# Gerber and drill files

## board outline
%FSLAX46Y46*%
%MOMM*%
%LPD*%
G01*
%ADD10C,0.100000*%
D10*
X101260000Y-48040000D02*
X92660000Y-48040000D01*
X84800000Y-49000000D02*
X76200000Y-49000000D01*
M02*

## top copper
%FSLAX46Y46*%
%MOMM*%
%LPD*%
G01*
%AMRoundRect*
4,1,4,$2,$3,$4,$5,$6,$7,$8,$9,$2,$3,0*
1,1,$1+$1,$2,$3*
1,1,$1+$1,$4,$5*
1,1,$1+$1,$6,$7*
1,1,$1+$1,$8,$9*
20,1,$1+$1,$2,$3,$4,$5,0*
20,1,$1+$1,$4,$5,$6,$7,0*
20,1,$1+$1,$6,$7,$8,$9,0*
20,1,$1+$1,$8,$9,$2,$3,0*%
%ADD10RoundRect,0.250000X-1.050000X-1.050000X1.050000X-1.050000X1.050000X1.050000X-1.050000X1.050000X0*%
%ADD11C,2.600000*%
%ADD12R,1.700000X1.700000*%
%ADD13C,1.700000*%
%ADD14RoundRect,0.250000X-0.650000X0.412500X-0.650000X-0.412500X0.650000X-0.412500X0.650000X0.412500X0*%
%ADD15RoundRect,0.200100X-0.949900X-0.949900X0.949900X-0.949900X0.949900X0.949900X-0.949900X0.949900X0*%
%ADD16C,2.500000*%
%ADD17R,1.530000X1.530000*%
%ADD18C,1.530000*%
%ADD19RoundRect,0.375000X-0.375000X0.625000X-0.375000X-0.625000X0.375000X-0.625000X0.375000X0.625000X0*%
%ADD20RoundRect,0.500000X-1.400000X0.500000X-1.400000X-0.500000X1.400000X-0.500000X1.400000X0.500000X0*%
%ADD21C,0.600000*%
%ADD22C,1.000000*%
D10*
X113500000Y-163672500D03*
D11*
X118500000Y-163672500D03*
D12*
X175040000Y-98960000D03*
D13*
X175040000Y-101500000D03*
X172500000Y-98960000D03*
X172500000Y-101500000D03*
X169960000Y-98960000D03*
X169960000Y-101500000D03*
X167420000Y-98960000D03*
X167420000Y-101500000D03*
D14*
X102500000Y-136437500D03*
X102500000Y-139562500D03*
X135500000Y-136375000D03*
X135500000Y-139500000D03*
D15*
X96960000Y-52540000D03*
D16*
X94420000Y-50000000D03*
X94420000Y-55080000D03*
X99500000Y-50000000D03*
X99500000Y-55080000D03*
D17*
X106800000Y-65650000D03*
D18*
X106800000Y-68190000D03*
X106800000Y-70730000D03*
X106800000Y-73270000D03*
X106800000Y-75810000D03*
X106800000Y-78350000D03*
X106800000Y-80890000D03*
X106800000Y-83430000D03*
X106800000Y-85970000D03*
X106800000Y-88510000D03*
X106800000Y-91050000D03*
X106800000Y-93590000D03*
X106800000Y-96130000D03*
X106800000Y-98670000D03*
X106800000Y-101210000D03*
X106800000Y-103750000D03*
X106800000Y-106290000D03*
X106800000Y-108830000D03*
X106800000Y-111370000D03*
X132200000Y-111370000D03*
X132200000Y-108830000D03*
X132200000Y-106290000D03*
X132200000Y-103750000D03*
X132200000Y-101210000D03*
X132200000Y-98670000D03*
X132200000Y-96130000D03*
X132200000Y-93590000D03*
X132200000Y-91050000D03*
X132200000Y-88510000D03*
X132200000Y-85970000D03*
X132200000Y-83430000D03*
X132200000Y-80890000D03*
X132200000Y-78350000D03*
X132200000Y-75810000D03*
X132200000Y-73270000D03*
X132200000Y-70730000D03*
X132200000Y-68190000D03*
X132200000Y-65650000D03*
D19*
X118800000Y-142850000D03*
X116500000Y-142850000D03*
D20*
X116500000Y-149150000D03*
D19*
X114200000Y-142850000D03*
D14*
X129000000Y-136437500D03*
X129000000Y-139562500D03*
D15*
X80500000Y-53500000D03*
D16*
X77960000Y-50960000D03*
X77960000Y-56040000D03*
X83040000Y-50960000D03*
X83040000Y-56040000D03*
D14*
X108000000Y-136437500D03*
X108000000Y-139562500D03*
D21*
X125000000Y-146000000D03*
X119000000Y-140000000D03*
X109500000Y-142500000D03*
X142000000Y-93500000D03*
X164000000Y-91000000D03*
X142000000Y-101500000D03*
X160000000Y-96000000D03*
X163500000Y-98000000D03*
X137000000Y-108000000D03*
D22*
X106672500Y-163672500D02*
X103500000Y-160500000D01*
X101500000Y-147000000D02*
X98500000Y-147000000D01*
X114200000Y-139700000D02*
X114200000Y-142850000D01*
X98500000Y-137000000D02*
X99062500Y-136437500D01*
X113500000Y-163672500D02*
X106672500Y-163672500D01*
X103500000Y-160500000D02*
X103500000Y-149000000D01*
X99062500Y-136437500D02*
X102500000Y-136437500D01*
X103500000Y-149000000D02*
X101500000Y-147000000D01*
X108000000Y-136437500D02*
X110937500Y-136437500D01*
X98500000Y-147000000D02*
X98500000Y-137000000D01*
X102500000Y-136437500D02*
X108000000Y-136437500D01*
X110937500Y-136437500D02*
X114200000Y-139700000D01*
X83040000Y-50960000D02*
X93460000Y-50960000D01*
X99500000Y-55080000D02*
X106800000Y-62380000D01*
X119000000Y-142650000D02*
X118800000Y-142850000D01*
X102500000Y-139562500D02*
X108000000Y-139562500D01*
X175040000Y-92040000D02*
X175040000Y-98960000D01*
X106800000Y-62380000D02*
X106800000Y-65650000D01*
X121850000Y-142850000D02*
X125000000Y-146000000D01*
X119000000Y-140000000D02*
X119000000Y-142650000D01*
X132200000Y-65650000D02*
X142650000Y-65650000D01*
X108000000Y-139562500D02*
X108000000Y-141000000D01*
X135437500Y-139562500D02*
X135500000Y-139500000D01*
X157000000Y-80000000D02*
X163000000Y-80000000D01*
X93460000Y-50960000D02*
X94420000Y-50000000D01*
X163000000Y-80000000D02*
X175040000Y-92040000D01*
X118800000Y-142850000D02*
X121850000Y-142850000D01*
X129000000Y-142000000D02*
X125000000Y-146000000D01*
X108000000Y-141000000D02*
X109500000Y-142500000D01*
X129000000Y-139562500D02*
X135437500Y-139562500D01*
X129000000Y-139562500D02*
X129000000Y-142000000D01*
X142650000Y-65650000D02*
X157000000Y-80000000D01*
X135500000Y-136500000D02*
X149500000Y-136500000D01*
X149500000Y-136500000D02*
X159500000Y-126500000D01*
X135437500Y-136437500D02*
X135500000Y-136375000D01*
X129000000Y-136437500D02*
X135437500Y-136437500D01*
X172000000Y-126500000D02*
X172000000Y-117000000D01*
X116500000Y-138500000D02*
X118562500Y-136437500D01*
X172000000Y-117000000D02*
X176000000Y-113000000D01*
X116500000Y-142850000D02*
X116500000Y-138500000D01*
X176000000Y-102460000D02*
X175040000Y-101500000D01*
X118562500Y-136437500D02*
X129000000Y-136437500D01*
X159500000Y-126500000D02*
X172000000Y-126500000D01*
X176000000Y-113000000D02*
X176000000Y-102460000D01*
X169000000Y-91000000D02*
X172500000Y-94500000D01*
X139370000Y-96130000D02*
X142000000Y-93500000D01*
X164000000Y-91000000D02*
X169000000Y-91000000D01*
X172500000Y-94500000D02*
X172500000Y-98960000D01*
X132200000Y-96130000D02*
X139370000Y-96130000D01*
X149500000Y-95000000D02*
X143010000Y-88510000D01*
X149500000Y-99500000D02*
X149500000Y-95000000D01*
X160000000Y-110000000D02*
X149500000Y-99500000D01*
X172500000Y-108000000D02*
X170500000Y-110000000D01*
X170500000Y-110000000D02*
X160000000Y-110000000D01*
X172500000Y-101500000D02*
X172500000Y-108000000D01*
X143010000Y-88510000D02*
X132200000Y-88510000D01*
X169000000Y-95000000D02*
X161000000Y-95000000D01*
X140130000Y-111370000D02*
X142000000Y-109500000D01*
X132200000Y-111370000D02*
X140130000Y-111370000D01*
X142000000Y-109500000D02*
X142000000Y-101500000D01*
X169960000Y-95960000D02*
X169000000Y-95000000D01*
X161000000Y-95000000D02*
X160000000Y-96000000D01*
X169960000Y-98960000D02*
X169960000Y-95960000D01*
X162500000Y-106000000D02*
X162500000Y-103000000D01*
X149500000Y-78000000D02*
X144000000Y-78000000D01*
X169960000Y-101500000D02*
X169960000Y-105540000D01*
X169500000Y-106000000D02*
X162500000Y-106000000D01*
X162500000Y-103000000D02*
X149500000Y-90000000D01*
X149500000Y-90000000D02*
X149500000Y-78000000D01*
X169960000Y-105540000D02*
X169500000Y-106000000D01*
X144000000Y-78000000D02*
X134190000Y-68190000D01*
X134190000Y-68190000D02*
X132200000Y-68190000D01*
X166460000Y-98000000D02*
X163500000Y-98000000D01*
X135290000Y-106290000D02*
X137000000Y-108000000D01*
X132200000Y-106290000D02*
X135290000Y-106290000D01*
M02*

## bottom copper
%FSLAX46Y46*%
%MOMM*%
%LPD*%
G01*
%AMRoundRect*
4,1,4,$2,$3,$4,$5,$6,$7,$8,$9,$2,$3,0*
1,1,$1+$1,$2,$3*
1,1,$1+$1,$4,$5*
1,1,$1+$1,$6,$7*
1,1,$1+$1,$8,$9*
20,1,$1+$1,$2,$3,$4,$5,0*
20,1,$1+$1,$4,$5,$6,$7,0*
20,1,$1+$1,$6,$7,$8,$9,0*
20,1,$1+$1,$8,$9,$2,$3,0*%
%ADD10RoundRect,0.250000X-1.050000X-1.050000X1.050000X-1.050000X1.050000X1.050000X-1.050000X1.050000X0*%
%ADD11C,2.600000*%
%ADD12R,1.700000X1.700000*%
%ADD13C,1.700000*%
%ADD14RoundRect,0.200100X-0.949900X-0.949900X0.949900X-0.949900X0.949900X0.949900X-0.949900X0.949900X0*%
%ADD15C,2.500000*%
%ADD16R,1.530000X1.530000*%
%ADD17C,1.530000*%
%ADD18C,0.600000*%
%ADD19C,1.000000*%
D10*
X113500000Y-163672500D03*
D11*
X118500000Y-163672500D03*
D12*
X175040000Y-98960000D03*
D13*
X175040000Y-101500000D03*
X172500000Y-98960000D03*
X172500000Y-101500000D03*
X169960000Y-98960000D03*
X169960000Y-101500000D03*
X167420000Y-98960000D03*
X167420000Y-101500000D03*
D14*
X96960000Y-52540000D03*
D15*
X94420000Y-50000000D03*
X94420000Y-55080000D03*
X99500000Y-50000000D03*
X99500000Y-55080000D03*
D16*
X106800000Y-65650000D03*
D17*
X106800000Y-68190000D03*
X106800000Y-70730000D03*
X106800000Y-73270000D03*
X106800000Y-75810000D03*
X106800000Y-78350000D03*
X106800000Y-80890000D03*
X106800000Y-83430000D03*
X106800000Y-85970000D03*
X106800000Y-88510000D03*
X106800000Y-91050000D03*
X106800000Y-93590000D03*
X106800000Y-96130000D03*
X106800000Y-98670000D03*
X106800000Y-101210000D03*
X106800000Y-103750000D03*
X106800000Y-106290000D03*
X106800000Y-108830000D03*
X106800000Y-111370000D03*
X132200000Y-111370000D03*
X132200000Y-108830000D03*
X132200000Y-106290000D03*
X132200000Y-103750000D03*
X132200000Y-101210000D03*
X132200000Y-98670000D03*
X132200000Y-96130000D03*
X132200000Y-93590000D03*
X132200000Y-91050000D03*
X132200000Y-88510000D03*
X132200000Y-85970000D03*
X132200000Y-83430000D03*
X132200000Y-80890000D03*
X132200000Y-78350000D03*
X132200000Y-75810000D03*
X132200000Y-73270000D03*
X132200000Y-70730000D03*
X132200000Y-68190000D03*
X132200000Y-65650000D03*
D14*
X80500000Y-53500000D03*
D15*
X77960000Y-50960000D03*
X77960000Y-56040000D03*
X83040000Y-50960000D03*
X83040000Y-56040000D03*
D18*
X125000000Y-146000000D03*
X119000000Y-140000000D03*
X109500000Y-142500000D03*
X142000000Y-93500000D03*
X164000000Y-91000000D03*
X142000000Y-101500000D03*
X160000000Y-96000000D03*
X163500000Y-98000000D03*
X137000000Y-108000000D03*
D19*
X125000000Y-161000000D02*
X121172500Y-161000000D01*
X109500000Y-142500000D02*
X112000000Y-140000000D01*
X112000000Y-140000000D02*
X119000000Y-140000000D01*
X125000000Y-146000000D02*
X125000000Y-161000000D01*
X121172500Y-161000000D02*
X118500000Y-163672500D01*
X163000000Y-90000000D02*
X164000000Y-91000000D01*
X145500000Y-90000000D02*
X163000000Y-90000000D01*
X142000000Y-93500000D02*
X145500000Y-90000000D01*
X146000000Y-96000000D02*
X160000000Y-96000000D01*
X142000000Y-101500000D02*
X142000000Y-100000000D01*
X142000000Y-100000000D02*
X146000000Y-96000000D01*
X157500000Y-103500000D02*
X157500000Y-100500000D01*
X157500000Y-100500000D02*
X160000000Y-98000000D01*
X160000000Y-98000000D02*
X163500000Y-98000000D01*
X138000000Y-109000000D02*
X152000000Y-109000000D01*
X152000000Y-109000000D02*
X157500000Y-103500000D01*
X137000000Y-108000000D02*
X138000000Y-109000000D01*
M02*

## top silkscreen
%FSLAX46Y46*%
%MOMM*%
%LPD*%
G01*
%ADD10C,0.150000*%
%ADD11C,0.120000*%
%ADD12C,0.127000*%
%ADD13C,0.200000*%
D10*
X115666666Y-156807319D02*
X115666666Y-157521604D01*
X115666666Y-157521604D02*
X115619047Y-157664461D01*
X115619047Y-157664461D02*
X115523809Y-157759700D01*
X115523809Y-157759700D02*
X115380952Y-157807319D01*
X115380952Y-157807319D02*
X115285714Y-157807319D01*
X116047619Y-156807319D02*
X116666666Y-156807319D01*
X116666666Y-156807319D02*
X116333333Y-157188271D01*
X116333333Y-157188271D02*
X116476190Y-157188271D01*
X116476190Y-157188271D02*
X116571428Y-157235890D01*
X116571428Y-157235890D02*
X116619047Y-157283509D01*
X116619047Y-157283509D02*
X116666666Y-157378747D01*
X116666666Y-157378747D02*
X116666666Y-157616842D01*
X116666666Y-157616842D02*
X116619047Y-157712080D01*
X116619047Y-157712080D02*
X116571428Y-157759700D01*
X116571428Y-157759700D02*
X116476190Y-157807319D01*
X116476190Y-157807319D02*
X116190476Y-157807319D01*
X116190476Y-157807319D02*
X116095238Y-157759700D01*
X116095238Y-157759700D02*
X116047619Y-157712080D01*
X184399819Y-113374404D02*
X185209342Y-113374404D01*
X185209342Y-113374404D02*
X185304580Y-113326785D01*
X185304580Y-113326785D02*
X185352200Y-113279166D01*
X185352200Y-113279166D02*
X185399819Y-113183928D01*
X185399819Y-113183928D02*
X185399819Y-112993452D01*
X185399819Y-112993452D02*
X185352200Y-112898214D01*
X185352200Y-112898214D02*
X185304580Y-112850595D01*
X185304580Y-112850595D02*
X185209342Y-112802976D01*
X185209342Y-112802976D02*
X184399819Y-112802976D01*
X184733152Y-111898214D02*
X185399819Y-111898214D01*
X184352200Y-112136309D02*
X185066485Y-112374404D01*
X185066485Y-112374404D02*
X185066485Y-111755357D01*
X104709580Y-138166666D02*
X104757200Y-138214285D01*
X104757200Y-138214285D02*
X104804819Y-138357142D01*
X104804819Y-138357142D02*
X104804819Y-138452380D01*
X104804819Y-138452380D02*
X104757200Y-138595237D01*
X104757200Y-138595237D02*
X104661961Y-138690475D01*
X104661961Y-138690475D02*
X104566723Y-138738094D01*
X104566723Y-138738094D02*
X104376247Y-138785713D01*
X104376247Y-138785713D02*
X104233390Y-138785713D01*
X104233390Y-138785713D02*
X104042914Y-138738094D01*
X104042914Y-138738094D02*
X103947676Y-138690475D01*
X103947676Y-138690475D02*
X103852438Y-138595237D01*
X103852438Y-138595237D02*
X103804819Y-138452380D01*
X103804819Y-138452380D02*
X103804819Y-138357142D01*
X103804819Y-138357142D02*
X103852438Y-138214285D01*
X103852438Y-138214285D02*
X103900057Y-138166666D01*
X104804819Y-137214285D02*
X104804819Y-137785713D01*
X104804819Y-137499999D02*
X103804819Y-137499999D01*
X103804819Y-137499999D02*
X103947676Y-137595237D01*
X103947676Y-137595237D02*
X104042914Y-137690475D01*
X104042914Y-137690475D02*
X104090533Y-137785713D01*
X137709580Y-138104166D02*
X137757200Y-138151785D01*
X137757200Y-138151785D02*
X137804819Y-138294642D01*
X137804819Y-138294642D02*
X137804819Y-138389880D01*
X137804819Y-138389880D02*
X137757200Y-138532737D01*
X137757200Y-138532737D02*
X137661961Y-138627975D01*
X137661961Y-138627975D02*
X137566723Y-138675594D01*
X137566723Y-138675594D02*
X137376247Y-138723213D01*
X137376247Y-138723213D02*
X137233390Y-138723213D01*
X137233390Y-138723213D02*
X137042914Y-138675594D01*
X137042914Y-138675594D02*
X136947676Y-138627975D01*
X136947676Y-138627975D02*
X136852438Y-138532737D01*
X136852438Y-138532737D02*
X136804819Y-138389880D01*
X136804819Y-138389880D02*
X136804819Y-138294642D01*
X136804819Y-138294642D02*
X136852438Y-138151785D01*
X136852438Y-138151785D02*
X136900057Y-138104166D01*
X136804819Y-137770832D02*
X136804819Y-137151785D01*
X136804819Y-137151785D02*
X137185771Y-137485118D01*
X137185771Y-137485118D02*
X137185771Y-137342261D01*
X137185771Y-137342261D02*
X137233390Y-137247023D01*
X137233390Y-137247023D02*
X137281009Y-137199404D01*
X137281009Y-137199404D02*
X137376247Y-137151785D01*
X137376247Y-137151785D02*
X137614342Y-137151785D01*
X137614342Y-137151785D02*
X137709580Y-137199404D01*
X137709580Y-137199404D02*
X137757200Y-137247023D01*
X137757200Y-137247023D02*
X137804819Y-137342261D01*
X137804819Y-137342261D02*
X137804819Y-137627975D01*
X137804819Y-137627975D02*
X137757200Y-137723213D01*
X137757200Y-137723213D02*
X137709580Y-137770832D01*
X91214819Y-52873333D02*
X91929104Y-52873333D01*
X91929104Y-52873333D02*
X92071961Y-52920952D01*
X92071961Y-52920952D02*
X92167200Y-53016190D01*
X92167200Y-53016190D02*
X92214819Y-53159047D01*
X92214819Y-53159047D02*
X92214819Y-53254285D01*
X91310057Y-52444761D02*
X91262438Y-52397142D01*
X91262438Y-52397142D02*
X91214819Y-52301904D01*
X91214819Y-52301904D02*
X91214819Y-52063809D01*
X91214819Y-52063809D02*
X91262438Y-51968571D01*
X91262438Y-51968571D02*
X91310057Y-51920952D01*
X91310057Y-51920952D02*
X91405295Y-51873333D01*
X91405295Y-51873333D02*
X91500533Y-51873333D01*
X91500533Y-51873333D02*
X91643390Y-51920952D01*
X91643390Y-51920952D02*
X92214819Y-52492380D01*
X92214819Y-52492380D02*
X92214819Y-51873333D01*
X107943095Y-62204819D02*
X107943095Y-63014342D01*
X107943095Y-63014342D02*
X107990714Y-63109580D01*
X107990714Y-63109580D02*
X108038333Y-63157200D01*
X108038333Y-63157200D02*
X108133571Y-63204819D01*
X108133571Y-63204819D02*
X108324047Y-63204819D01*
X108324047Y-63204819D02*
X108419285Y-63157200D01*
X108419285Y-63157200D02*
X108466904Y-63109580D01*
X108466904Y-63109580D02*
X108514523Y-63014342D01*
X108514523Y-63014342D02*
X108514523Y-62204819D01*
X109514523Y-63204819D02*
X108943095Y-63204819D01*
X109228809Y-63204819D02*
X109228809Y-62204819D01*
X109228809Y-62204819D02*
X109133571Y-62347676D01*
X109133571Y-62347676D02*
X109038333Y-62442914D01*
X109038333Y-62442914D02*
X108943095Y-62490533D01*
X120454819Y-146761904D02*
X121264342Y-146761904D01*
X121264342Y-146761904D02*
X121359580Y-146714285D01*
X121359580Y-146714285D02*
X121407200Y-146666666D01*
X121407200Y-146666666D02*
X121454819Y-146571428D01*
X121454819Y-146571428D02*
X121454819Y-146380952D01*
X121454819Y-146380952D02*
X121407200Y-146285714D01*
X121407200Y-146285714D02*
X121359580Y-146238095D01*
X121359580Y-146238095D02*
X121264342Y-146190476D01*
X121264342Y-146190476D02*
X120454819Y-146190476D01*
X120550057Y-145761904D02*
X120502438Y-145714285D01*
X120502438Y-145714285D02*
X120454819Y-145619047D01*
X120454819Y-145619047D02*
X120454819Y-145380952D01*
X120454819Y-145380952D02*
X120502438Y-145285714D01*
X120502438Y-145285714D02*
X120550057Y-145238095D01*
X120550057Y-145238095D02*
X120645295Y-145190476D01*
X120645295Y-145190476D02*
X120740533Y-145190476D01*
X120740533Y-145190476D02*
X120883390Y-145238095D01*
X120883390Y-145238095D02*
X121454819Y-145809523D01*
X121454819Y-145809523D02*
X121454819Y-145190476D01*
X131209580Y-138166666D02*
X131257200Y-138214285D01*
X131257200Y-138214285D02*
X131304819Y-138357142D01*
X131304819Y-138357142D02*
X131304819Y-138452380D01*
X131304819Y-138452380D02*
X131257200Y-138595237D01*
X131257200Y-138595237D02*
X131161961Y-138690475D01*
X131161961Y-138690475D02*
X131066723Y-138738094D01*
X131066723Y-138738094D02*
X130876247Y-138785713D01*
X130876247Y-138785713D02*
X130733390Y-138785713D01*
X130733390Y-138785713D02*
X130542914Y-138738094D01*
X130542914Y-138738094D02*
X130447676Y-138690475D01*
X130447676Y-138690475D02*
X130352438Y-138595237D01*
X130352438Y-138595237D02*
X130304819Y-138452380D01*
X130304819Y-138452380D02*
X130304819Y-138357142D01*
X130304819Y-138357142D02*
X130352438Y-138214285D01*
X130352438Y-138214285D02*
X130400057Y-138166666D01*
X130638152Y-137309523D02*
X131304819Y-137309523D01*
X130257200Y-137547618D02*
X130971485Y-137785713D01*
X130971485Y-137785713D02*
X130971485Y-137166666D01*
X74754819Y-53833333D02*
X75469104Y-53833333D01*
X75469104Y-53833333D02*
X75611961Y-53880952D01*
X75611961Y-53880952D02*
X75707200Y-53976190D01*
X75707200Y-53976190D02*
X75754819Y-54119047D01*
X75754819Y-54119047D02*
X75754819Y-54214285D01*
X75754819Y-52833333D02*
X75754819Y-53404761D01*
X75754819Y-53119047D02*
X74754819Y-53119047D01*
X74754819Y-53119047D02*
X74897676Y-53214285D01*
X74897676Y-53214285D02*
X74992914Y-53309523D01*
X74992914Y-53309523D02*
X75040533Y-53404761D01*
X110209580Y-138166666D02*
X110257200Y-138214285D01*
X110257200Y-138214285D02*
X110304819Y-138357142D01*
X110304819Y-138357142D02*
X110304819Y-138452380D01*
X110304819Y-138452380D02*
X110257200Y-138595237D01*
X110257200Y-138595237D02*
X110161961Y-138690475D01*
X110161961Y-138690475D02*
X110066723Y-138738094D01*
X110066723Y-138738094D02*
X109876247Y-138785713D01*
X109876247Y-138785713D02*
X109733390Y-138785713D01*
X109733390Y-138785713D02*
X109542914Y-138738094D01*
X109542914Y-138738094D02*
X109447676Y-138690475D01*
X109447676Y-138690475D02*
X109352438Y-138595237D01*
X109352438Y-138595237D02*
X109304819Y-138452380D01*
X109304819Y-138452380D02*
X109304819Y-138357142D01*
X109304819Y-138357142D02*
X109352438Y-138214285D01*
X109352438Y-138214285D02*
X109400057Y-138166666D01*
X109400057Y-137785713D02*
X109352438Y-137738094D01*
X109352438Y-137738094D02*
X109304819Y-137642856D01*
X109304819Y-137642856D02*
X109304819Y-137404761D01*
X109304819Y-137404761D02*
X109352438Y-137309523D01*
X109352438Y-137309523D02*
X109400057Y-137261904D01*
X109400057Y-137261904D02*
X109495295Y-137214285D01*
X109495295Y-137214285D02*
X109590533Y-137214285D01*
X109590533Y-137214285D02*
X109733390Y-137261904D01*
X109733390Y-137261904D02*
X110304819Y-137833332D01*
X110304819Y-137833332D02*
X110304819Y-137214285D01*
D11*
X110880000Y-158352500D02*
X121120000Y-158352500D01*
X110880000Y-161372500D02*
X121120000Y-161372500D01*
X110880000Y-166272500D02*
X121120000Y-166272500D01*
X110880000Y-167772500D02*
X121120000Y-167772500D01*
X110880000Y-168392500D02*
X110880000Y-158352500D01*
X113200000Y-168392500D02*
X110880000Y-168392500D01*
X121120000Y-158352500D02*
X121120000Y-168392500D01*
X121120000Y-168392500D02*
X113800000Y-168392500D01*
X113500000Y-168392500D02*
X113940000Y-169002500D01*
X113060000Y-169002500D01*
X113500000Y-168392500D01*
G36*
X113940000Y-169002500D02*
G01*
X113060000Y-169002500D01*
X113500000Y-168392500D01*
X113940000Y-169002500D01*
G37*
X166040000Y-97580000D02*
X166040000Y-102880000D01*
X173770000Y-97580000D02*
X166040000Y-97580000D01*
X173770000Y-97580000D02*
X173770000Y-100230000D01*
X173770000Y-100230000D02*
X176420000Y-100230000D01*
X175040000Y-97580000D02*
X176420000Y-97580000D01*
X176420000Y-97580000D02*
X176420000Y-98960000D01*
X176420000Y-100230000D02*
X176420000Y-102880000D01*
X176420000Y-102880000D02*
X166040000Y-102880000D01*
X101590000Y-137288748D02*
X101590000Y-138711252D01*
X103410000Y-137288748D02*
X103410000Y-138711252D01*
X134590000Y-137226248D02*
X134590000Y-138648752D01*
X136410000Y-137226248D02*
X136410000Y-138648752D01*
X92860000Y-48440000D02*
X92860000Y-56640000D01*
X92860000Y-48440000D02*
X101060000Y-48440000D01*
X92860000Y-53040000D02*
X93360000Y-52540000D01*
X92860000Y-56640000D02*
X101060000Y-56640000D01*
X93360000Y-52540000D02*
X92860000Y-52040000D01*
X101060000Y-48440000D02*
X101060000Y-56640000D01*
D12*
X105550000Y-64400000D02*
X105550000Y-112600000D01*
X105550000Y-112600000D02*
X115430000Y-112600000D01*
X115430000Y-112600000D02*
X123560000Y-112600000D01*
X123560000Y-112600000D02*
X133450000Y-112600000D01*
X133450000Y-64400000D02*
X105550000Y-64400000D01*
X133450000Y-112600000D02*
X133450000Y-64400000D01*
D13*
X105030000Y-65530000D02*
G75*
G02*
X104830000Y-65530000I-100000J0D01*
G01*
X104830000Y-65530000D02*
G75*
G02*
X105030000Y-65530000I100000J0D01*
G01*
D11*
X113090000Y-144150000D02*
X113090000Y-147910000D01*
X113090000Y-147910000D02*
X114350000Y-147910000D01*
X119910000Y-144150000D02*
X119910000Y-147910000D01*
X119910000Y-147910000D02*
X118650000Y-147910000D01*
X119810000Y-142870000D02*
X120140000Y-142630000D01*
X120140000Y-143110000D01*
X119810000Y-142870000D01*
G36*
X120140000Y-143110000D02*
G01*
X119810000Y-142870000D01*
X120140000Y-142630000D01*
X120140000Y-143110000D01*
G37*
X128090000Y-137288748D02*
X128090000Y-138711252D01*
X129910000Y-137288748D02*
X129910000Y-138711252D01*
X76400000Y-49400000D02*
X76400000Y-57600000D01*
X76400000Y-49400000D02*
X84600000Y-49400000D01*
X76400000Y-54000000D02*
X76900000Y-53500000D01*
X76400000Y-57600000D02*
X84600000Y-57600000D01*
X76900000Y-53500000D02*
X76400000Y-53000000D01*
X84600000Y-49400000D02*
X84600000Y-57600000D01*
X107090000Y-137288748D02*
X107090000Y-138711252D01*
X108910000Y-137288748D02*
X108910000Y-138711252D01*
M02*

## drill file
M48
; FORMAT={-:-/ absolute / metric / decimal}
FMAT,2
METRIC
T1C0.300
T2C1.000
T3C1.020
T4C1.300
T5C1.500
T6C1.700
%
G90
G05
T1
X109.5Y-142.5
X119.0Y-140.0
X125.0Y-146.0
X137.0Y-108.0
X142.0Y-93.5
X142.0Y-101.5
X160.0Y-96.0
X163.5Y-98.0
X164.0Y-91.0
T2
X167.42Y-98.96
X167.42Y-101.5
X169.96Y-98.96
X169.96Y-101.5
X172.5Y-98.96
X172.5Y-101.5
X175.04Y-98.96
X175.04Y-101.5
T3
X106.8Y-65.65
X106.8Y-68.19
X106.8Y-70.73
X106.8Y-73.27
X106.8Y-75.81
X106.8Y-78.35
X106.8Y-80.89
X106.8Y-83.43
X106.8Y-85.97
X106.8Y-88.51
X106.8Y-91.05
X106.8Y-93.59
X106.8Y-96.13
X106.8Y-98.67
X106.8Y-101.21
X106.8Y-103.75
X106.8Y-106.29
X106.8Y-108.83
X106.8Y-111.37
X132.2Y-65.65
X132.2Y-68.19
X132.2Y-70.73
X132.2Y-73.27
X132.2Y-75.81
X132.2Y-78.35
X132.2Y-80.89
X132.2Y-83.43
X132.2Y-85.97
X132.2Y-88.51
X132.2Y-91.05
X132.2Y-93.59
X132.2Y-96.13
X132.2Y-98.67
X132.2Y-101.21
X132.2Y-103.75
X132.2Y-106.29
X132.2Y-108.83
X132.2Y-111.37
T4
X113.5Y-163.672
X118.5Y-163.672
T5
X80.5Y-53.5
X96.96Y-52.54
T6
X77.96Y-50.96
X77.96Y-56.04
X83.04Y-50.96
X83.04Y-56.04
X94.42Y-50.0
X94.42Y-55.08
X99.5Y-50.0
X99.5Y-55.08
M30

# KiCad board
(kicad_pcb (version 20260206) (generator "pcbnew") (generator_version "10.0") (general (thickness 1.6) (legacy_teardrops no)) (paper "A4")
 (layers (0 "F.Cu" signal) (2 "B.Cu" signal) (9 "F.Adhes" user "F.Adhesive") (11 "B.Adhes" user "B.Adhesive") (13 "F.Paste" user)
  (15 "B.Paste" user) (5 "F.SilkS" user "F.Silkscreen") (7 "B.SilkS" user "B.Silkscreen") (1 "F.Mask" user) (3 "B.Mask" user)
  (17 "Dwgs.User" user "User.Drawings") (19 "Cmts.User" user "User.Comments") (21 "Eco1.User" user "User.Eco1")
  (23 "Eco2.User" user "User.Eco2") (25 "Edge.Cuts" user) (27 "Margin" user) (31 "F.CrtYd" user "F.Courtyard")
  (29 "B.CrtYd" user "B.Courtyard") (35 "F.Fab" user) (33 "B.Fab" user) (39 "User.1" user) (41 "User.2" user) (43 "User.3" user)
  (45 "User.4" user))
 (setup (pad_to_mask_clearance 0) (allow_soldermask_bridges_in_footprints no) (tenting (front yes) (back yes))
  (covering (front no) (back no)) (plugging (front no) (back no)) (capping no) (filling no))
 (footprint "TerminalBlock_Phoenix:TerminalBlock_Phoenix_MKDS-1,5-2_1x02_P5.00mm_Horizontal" (layer "F.Cu") (at 113.5 163.6725)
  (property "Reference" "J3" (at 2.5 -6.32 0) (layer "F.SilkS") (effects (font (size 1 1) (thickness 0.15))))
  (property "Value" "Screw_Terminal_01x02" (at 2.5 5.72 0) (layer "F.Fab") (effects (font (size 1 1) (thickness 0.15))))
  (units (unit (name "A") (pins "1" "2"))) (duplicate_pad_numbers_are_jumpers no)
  (fp_line (start -2.62 -5.32) (end 7.62 -5.32) (stroke (width 0.12) (type solid)) (layer "F.SilkS"))
  (fp_line (start -2.62 -2.3) (end 7.62 -2.3) (stroke (width 0.12) (type solid)) (layer "F.SilkS"))
  (fp_line (start -2.62 2.6) (end 7.62 2.6) (stroke (width 0.12) (type solid)) (layer "F.SilkS"))
  (fp_line (start -2.62 4.1) (end 7.62 4.1) (stroke (width 0.12) (type solid)) (layer "F.SilkS"))
  (fp_line (start -2.62 4.72) (end -2.62 -5.32) (stroke (width 0.12) (type solid)) (layer "F.SilkS"))
  (fp_line (start -0.3 4.72) (end -2.62 4.72) (stroke (width 0.12) (type solid)) (layer "F.SilkS"))
  (fp_line (start 7.62 -5.32) (end 7.62 4.72) (stroke (width 0.12) (type solid)) (layer "F.SilkS"))
  (fp_line (start 7.62 4.72) (end 0.3 4.72) (stroke (width 0.12) (type solid)) (layer "F.SilkS"))
  (fp_poly (pts (xy 0 4.72) (xy 0.44 5.33) (xy -0.44 5.33)) (stroke (width 0.12) (type solid)) (fill yes) (layer "F.SilkS"))
  (pad "1" thru_hole roundrect (at 0 0) (size 2.6 2.6) (drill 1.3) (layers "*.Cu" "*.Mask") (remove_unused_layers no)
   (roundrect_rratio 0.096154) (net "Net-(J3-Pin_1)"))
  (pad "2" thru_hole circle (at 5 0) (size 2.6 2.6) (drill 1.3) (layers "*.Cu" "*.Mask") (remove_unused_layers no) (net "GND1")))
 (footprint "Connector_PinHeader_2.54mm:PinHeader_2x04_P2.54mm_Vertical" (layer "F.Cu") (at 175.04 98.96 -90)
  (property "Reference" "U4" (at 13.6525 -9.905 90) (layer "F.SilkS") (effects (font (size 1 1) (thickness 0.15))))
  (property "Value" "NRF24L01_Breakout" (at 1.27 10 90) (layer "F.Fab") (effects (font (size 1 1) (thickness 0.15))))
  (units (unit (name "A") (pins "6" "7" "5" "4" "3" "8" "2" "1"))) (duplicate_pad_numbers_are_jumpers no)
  (fp_line (start -1.38 9) (end 3.92 9) (stroke (width 0.12) (type solid)) (layer "F.SilkS"))
  (fp_line (start -1.38 1.27) (end -1.38 9) (stroke (width 0.12) (type solid)) (layer "F.SilkS"))
  (fp_line (start -1.38 1.27) (end 1.27 1.27) (stroke (width 0.12) (type solid)) (layer "F.SilkS"))
  (fp_line (start 1.27 1.27) (end 1.27 -1.38) (stroke (width 0.12) (type solid)) (layer "F.SilkS"))
  (fp_line (start -1.38 0) (end -1.38 -1.38) (stroke (width 0.12) (type solid)) (layer "F.SilkS"))
  (fp_line (start -1.38 -1.38) (end 0 -1.38) (stroke (width 0.12) (type solid)) (layer "F.SilkS"))
  (fp_line (start 1.27 -1.38) (end 3.92 -1.38) (stroke (width 0.12) (type solid)) (layer "F.SilkS"))
  (fp_line (start 3.92 -1.38) (end 3.92 9) (stroke (width 0.12) (type solid)) (layer "F.SilkS"))
  (pad "1" thru_hole rect (at 0 0 270) (size 1.7 1.7) (drill 1) (layers "*.Cu" "*.Mask") (remove_unused_layers no) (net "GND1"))
  (pad "2" thru_hole circle (at 2.54 0 270) (size 1.7 1.7) (drill 1) (layers "*.Cu" "*.Mask") (remove_unused_layers no) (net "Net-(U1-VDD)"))
  (pad "3" thru_hole circle (at 0 2.54 270) (size 1.7 1.7) (drill 1) (layers "*.Cu" "*.Mask") (remove_unused_layers no) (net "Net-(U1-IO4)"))
  (pad "4" thru_hole circle (at 2.54 2.54 270) (size 1.7 1.7) (drill 1) (layers "*.Cu" "*.Mask") (remove_unused_layers no)
   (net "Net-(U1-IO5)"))
  (pad "5" thru_hole circle (at 0 5.08 270) (size 1.7 1.7) (drill 1) (layers "*.Cu" "*.Mask") (remove_unused_layers no)
   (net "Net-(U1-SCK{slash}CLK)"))
  (pad "6" thru_hole circle (at 2.54 5.08 270) (size 1.7 1.7) (drill 1) (layers "*.Cu" "*.Mask") (remove_unused_layers no)
   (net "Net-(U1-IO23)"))
  (pad "7" thru_hole circle (at 0 7.62 270) (size 1.7 1.7) (drill 1) (layers "*.Cu" "*.Mask") (remove_unused_layers no)
   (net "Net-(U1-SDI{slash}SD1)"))
  (pad "8" thru_hole circle (at 2.54 7.62 270) (size 1.7 1.7) (drill 1) (layers "*.Cu" "*.Mask") (remove_unused_layers no)
   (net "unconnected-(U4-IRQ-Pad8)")))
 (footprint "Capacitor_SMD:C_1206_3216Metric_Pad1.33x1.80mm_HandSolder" (layer "F.Cu") (at 102.5 138 -90)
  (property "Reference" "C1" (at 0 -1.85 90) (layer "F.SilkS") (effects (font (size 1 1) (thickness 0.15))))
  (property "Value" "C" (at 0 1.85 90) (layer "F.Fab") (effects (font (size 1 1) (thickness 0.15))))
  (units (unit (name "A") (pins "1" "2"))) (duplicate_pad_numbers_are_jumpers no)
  (fp_line (start -0.711252 0.91) (end 0.711252 0.91) (stroke (width 0.12) (type solid)) (layer "F.SilkS"))
  (fp_line (start -0.711252 -0.91) (end 0.711252 -0.91) (stroke (width 0.12) (type solid)) (layer "F.SilkS"))
  (pad "1" smd roundrect (at -1.5625 0 270) (size 1.325 1.8) (layers "F.Cu" "F.Mask" "F.Paste") (roundrect_rratio 0.188679)
   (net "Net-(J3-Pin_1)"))
  (pad "2" smd roundrect (at 1.5625 0 270) (size 1.325 1.8) (layers "F.Cu" "F.Mask" "F.Paste") (roundrect_rratio 0.188679) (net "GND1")))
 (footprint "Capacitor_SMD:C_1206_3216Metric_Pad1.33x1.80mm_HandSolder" (layer "F.Cu") (at 135.5 137.9375 -90)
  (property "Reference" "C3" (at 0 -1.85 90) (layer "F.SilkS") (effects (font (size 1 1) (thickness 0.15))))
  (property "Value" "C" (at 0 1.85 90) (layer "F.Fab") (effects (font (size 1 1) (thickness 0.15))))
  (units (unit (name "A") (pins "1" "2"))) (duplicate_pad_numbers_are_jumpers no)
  (fp_line (start -0.711252 0.91) (end 0.711252 0.91) (stroke (width 0.12) (type solid)) (layer "F.SilkS"))
  (fp_line (start -0.711252 -0.91) (end 0.711252 -0.91) (stroke (width 0.12) (type solid)) (layer "F.SilkS"))
  (pad "1" smd roundrect (at -1.5625 0 270) (size 1.325 1.8) (layers "F.Cu" "F.Mask" "F.Paste") (roundrect_rratio 0.188679)
   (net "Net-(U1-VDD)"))
  (pad "2" smd roundrect (at 1.5625 0 270) (size 1.325 1.8) (layers "F.Cu" "F.Mask" "F.Paste") (roundrect_rratio 0.188679) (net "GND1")))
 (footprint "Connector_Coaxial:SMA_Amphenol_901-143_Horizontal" (layer "F.Cu") (at 96.96 52.54)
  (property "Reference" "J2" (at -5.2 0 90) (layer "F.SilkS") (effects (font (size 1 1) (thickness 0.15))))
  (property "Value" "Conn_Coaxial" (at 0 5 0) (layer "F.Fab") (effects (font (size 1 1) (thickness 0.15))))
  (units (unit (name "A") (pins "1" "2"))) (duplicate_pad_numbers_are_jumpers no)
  (fp_line (start -4.1 -4.1) (end -4.1 4.1) (stroke (width 0.12) (type solid)) (layer "F.SilkS"))
  (fp_line (start -4.1 -4.1) (end 4.1 -4.1) (stroke (width 0.12) (type solid)) (layer "F.SilkS"))
  (fp_line (start -4.1 0.5) (end -3.6 0) (stroke (width 0.12) (type solid)) (layer "F.SilkS"))
  (fp_line (start -4.1 4.1) (end 4.1 4.1) (stroke (width 0.12) (type solid)) (layer "F.SilkS"))
  (fp_line (start -3.6 0) (end -4.1 -0.5) (stroke (width 0.12) (type solid)) (layer "F.SilkS"))
  (fp_line (start 4.1 -4.1) (end 4.1 4.1) (stroke (width 0.12) (type solid)) (layer "F.SilkS"))
  (fp_line (start 4.3 -4.5) (end -4.3 -4.5) (stroke (width 0.1) (type solid)) (layer "Edge.Cuts"))
  (pad "1" thru_hole roundrect (at 0 0) (size 2.3 2.3) (drill 1.5) (layers "*.Cu" "*.Mask") (remove_unused_layers yes) (keep_end_layers yes)
   (zone_layer_connections) (roundrect_rratio 0.087) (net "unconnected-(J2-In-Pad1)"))
  (pad "2" thru_hole circle (at -2.54 -2.54) (size 2.5 2.5) (drill 1.7) (layers "*.Cu" "*.Mask") (remove_unused_layers yes)
   (keep_end_layers yes) (zone_layer_connections) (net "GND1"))
  (pad "2" thru_hole circle (at -2.54 2.54) (size 2.5 2.5) (drill 1.7) (layers "*.Cu" "*.Mask") (remove_unused_layers yes)
   (keep_end_layers yes) (zone_layer_connections) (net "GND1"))
  (pad "2" thru_hole circle (at 2.54 -2.54) (size 2.5 2.5) (drill 1.7) (layers "*.Cu" "*.Mask") (remove_unused_layers yes)
   (keep_end_layers yes) (zone_layer_connections) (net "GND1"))
  (pad "2" thru_hole circle (at 2.54 2.54) (size 2.5 2.5) (drill 1.7) (layers "*.Cu" "*.Mask") (remove_unused_layers yes)
   (keep_end_layers yes) (zone_layer_connections) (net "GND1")))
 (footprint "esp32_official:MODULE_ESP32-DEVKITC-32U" (layer "F.Cu") (at 119.5 88.5)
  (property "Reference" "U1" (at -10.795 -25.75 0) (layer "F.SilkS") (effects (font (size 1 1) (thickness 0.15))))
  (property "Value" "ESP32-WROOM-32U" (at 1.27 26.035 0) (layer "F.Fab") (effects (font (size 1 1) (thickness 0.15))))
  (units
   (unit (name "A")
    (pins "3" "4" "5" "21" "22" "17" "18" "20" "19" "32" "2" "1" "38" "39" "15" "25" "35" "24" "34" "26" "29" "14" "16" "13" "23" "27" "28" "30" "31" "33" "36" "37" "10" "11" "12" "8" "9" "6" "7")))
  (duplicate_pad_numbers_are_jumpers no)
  (fp_line (start -13.95 -24.1) (end -13.95 24.1) (stroke (width 0.127) (type solid)) (layer "F.SilkS"))
  (fp_line (start -13.95 24.1) (end -4.07 24.1) (stroke (width 0.127) (type solid)) (layer "F.SilkS"))
  (fp_line (start -4.07 24.1) (end 4.06 24.1) (stroke (width 0.127) (type solid)) (layer "F.SilkS"))
  (fp_line (start 4.06 24.1) (end 13.95 24.1) (stroke (width 0.127) (type solid)) (layer "F.SilkS"))
  (fp_line (start 13.95 -24.1) (end -13.95 -24.1) (stroke (width 0.127) (type solid)) (layer "F.SilkS"))
  (fp_line (start 13.95 24.1) (end 13.95 -24.1) (stroke (width 0.127) (type solid)) (layer "F.SilkS"))
  (fp_circle (center -14.57 -22.97) (end -14.47 -22.97) (stroke (width 0.2) (type solid)) (fill no) (layer "F.SilkS"))
  (pad "1" thru_hole rect (at -12.7 -22.85) (size 1.53 1.53) (drill 1.02) (layers "*.Cu" "*.Mask") (remove_unused_layers no) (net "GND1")
   (solder_mask_margin 0.102))
  (pad "2" thru_hole circle (at -12.7 -20.31) (size 1.53 1.53) (drill 1.02) (layers "*.Cu" "*.Mask") (remove_unused_layers no)
   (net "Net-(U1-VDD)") (solder_mask_margin 0.102))
  (pad "3" thru_hole circle (at -12.7 -17.77) (size 1.53 1.53) (drill 1.02) (layers "*.Cu" "*.Mask") (remove_unused_layers no)
   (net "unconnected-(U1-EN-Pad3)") (solder_mask_margin 0.102))
  (pad "4" thru_hole circle (at -12.7 -15.23) (size 1.53 1.53) (drill 1.02) (layers "*.Cu" "*.Mask") (remove_unused_layers no)
   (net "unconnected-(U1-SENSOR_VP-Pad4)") (solder_mask_margin 0.102))
  (pad "5" thru_hole circle (at -12.7 -12.69) (size 1.53 1.53) (drill 1.02) (layers "*.Cu" "*.Mask") (remove_unused_layers no)
   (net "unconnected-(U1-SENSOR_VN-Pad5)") (solder_mask_margin 0.102))
  (pad "6" thru_hole circle (at -12.7 -10.15) (size 1.53 1.53) (drill 1.02) (layers "*.Cu" "*.Mask") (remove_unused_layers no)
   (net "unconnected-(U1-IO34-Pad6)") (solder_mask_margin 0.102))
  (pad "7" thru_hole circle (at -12.7 -7.61) (size 1.53 1.53) (drill 1.02) (layers "*.Cu" "*.Mask") (remove_unused_layers no)
   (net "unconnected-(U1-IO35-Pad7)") (solder_mask_margin 0.102))
  (pad "8" thru_hole circle (at -12.7 -5.07) (size 1.53 1.53) (drill 1.02) (layers "*.Cu" "*.Mask") (remove_unused_layers no)
   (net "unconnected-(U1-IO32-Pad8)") (solder_mask_margin 0.102))
  (pad "9" thru_hole circle (at -12.7 -2.53) (size 1.53 1.53) (drill 1.02) (layers "*.Cu" "*.Mask") (remove_unused_layers no)
   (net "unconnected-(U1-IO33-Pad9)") (solder_mask_margin 0.102))
  (pad "10" thru_hole circle (at -12.7 0.01) (size 1.53 1.53) (drill 1.02) (layers "*.Cu" "*.Mask") (remove_unused_layers no)
   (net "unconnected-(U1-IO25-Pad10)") (solder_mask_margin 0.102))
  (pad "11" thru_hole circle (at -12.7 2.55) (size 1.53 1.53) (drill 1.02) (layers "*.Cu" "*.Mask") (remove_unused_layers no)
   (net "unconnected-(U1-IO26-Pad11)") (solder_mask_margin 0.102))
  (pad "12" thru_hole circle (at -12.7 5.09) (size 1.53 1.53) (drill 1.02) (layers "*.Cu" "*.Mask") (remove_unused_layers no)
   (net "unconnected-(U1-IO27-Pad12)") (solder_mask_margin 0.102))
  (pad "13" thru_hole circle (at -12.7 7.63) (size 1.53 1.53) (drill 1.02) (layers "*.Cu" "*.Mask") (remove_unused_layers no)
   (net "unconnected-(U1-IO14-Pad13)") (solder_mask_margin 0.102))
  (pad "14" thru_hole circle (at -12.7 10.17) (size 1.53 1.53) (drill 1.02) (layers "*.Cu" "*.Mask") (remove_unused_layers no)
   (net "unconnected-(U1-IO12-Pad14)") (solder_mask_margin 0.102))
  (pad "15" thru_hole circle (at -12.7 12.71) (size 1.53 1.53) (drill 1.02) (layers "*.Cu" "*.Mask") (remove_unused_layers no) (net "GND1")
   (solder_mask_margin 0.102))
  (pad "16" thru_hole circle (at -12.7 15.25) (size 1.53 1.53) (drill 1.02) (layers "*.Cu" "*.Mask") (remove_unused_layers no)
   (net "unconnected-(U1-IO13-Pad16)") (solder_mask_margin 0.102))
  (pad "17" thru_hole circle (at -12.7 17.79) (size 1.53 1.53) (drill 1.02) (layers "*.Cu" "*.Mask") (remove_unused_layers no)
   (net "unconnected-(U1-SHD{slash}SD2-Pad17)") (solder_mask_margin 0.102))
  (pad "18" thru_hole circle (at -12.7 20.33) (size 1.53 1.53) (drill 1.02) (layers "*.Cu" "*.Mask") (remove_unused_layers no)
   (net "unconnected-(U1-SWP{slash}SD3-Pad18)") (solder_mask_margin 0.102))
  (pad "19" thru_hole circle (at -12.7 22.87) (size 1.53 1.53) (drill 1.02) (layers "*.Cu" "*.Mask") (remove_unused_layers no)
   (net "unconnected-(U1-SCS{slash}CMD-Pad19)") (solder_mask_margin 0.102))
  (pad "20" thru_hole circle (at 12.7 22.87) (size 1.53 1.53) (drill 1.02) (layers "*.Cu" "*.Mask") (remove_unused_layers no)
   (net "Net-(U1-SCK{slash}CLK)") (solder_mask_margin 0.102))
  (pad "21" thru_hole circle (at 12.7 20.33) (size 1.53 1.53) (drill 1.02) (layers "*.Cu" "*.Mask") (remove_unused_layers no)
   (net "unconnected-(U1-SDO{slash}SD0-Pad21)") (solder_mask_margin 0.102))
  (pad "22" thru_hole circle (at 12.7 17.79) (size 1.53 1.53) (drill 1.02) (layers "*.Cu" "*.Mask") (remove_unused_layers no)
   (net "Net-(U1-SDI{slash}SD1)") (solder_mask_margin 0.102))
  (pad "23" thru_hole circle (at 12.7 15.25) (size 1.53 1.53) (drill 1.02) (layers "*.Cu" "*.Mask") (remove_unused_layers no)
   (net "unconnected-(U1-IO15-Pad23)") (solder_mask_margin 0.102))
  (pad "24" thru_hole circle (at 12.7 12.71) (size 1.53 1.53) (drill 1.02) (layers "*.Cu" "*.Mask") (remove_unused_layers no)
   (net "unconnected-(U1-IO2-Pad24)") (solder_mask_margin 0.102))
  (pad "25" thru_hole circle (at 12.7 10.17) (size 1.53 1.53) (drill 1.02) (layers "*.Cu" "*.Mask") (remove_unused_layers no)
   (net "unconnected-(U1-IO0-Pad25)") (solder_mask_margin 0.102))
  (pad "26" thru_hole circle (at 12.7 7.63) (size 1.53 1.53) (drill 1.02) (layers "*.Cu" "*.Mask") (remove_unused_layers no)
   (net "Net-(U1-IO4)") (solder_mask_margin 0.102))
  (pad "27" thru_hole circle (at 12.7 5.09) (size 1.53 1.53) (drill 1.02) (layers "*.Cu" "*.Mask") (remove_unused_layers no)
   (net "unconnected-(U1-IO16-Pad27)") (solder_mask_margin 0.102))
  (pad "28" thru_hole circle (at 12.7 2.55) (size 1.53 1.53) (drill 1.02) (layers "*.Cu" "*.Mask") (remove_unused_layers no)
   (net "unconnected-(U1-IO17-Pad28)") (solder_mask_margin 0.102))
  (pad "29" thru_hole circle (at 12.7 0.01) (size 1.53 1.53) (drill 1.02) (layers "*.Cu" "*.Mask") (remove_unused_layers no)
   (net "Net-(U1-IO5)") (solder_mask_margin 0.102))
  (pad "30" thru_hole circle (at 12.7 -2.53) (size 1.53 1.53) (drill 1.02) (layers "*.Cu" "*.Mask") (remove_unused_layers no)
   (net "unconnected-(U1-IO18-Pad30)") (solder_mask_margin 0.102))
  (pad "31" thru_hole circle (at 12.7 -5.07) (size 1.53 1.53) (drill 1.02) (layers "*.Cu" "*.Mask") (remove_unused_layers no)
   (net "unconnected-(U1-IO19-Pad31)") (solder_mask_margin 0.102))
  (pad "32" thru_hole circle (at 12.7 -7.61) (size 1.53 1.53) (drill 1.02) (layers "*.Cu" "*.Mask") (remove_unused_layers no)
   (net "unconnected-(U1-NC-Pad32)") (solder_mask_margin 0.102))
  (pad "33" thru_hole circle (at 12.7 -10.15) (size 1.53 1.53) (drill 1.02) (layers "*.Cu" "*.Mask") (remove_unused_layers no)
   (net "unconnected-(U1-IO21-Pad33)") (solder_mask_margin 0.102))
  (pad "34" thru_hole circle (at 12.7 -12.69) (size 1.53 1.53) (drill 1.02) (layers "*.Cu" "*.Mask") (remove_unused_layers no)
   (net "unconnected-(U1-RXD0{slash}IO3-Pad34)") (solder_mask_margin 0.102))
  (pad "35" thru_hole circle (at 12.7 -15.23) (size 1.53 1.53) (drill 1.02) (layers "*.Cu" "*.Mask") (remove_unused_layers no)
   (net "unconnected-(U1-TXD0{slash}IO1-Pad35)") (solder_mask_margin 0.102))
  (pad "36" thru_hole circle (at 12.7 -17.77) (size 1.53 1.53) (drill 1.02) (layers "*.Cu" "*.Mask") (remove_unused_layers no)
   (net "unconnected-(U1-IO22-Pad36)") (solder_mask_margin 0.102))
  (pad "37" thru_hole circle (at 12.7 -20.31) (size 1.53 1.53) (drill 1.02) (layers "*.Cu" "*.Mask") (remove_unused_layers no)
   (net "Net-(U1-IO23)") (solder_mask_margin 0.102))
  (pad "38" thru_hole circle (at 12.7 -22.85) (size 1.53 1.53) (drill 1.02) (layers "*.Cu" "*.Mask") (remove_unused_layers no) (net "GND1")
   (solder_mask_margin 0.102)))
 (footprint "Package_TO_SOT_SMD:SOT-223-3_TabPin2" (layer "F.Cu") (at 116.5 146 -90)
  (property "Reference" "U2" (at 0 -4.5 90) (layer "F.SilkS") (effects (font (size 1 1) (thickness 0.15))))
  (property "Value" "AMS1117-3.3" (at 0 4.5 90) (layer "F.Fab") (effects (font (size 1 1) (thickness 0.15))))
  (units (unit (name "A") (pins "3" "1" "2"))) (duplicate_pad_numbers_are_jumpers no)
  (fp_line (start -1.85 3.41) (end 1.91 3.41) (stroke (width 0.12) (type solid)) (layer "F.SilkS"))
  (fp_line (start 1.91 3.41) (end 1.91 2.15) (stroke (width 0.12) (type solid)) (layer "F.SilkS"))
  (fp_line (start -1.85 -3.41) (end 1.91 -3.41) (stroke (width 0.12) (type solid)) (layer "F.SilkS"))
  (fp_line (start 1.91 -3.41) (end 1.91 -2.15) (stroke (width 0.12) (type solid)) (layer "F.SilkS"))
  (fp_poly
   (pts (xy -3.13 -3.31) (xy -3.37 -3.64) (xy -2.89 -3.64) (xy -3.13 -3.31)) (stroke (width 0.12) (type solid)) (fill yes) (layer "F.SilkS"))
  (pad "1" smd roundrect (at -3.15 -2.3 270) (size 2 1.5) (layers "F.Cu" "F.Mask" "F.Paste") (roundrect_rratio 0.25) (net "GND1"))
  (pad "2" smd roundrect (at -3.15 0 270) (size 2 1.5) (layers "F.Cu" "F.Mask" "F.Paste") (roundrect_rratio 0.25) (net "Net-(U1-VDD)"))
  (pad "2" smd roundrect (at 3.15 0 270) (size 2 3.8) (layers "F.Cu" "F.Mask" "F.Paste") (roundrect_rratio 0.25) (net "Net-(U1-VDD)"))
  (pad "3" smd roundrect (at -3.15 2.3 270) (size 2 1.5) (layers "F.Cu" "F.Mask" "F.Paste") (roundrect_rratio 0.25) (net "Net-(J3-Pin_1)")))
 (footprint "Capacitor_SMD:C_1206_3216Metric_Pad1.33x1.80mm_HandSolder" (layer "F.Cu") (at 129 138 -90)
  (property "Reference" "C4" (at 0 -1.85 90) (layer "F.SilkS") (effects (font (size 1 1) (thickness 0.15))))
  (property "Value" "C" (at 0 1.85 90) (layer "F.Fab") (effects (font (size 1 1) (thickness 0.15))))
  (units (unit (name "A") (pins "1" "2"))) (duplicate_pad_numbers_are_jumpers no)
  (fp_line (start -0.711252 0.91) (end 0.711252 0.91) (stroke (width 0.12) (type solid)) (layer "F.SilkS"))
  (fp_line (start -0.711252 -0.91) (end 0.711252 -0.91) (stroke (width 0.12) (type solid)) (layer "F.SilkS"))
  (pad "1" smd roundrect (at -1.5625 0 270) (size 1.325 1.8) (layers "F.Cu" "F.Mask" "F.Paste") (roundrect_rratio 0.188679)
   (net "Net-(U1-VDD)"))
  (pad "2" smd roundrect (at 1.5625 0 270) (size 1.325 1.8) (layers "F.Cu" "F.Mask" "F.Paste") (roundrect_rratio 0.188679) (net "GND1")))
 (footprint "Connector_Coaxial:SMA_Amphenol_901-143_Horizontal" (layer "F.Cu") (at 80.5 53.5)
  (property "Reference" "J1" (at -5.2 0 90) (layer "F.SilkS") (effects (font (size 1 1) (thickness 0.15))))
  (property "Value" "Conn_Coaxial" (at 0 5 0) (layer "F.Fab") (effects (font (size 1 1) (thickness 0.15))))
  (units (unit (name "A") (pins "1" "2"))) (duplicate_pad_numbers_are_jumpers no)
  (fp_line (start -4.1 -4.1) (end -4.1 4.1) (stroke (width 0.12) (type solid)) (layer "F.SilkS"))
  (fp_line (start -4.1 -4.1) (end 4.1 -4.1) (stroke (width 0.12) (type solid)) (layer "F.SilkS"))
  (fp_line (start -4.1 0.5) (end -3.6 0) (stroke (width 0.12) (type solid)) (layer "F.SilkS"))
  (fp_line (start -4.1 4.1) (end 4.1 4.1) (stroke (width 0.12) (type solid)) (layer "F.SilkS"))
  (fp_line (start -3.6 0) (end -4.1 -0.5) (stroke (width 0.12) (type solid)) (layer "F.SilkS"))
  (fp_line (start 4.1 -4.1) (end 4.1 4.1) (stroke (width 0.12) (type solid)) (layer "F.SilkS"))
  (fp_line (start 4.3 -4.5) (end -4.3 -4.5) (stroke (width 0.1) (type solid)) (layer "Edge.Cuts"))
  (pad "1" thru_hole roundrect (at 0 0) (size 2.3 2.3) (drill 1.5) (layers "*.Cu" "*.Mask") (remove_unused_layers yes) (keep_end_layers yes)
   (zone_layer_connections) (roundrect_rratio 0.087) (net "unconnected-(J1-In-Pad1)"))
  (pad "2" thru_hole circle (at -2.54 -2.54) (size 2.5 2.5) (drill 1.7) (layers "*.Cu" "*.Mask") (remove_unused_layers yes)
   (keep_end_layers yes) (zone_layer_connections) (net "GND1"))
  (pad "2" thru_hole circle (at -2.54 2.54) (size 2.5 2.5) (drill 1.7) (layers "*.Cu" "*.Mask") (remove_unused_layers yes)
   (keep_end_layers yes) (zone_layer_connections) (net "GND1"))
  (pad "2" thru_hole circle (at 2.54 -2.54) (size 2.5 2.5) (drill 1.7) (layers "*.Cu" "*.Mask") (remove_unused_layers yes)
   (keep_end_layers yes) (zone_layer_connections) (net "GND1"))
  (pad "2" thru_hole circle (at 2.54 2.54) (size 2.5 2.5) (drill 1.7) (layers "*.Cu" "*.Mask") (remove_unused_layers yes)
   (keep_end_layers yes) (zone_layer_connections) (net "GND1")))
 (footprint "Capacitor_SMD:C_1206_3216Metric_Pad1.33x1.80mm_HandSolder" (layer "F.Cu") (at 108 138 -90)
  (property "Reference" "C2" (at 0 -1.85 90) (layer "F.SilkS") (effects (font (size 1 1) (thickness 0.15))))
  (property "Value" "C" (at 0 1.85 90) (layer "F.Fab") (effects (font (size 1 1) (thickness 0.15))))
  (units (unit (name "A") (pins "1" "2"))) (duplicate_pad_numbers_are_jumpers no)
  (fp_line (start -0.711252 0.91) (end 0.711252 0.91) (stroke (width 0.12) (type solid)) (layer "F.SilkS"))
  (fp_line (start -0.711252 -0.91) (end 0.711252 -0.91) (stroke (width 0.12) (type solid)) (layer "F.SilkS"))
  (pad "1" smd roundrect (at -1.5625 0 270) (size 1.325 1.8) (layers "F.Cu" "F.Mask" "F.Paste") (roundrect_rratio 0.188679)
   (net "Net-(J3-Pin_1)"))
  (pad "2" smd roundrect (at 1.5625 0 270) (size 1.325 1.8) (layers "F.Cu" "F.Mask" "F.Paste") (roundrect_rratio 0.188679) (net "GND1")))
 (segment (start 106.6725 163.6725) (end 103.5 160.5) (width 1) (layer "F.Cu") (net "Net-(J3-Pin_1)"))
 (segment (start 101.5 147) (end 98.5 147) (width 1) (layer "F.Cu") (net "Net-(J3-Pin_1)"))
 (segment (start 114.2 139.7) (end 114.2 142.85) (width 1) (layer "F.Cu") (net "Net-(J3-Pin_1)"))
 (segment (start 98.5 137) (end 99.0625 136.4375) (width 1) (layer "F.Cu") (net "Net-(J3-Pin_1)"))
 (segment (start 113.5 163.6725) (end 106.6725 163.6725) (width 1) (layer "F.Cu") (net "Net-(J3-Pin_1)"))
 (segment (start 103.5 160.5) (end 103.5 149) (width 1) (layer "F.Cu") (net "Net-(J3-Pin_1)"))
 (segment (start 99.0625 136.4375) (end 102.5 136.4375) (width 1) (layer "F.Cu") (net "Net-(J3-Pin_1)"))
 (segment (start 103.5 149) (end 101.5 147) (width 1) (layer "F.Cu") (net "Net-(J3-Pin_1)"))
 (segment (start 108 136.4375) (end 110.9375 136.4375) (width 1) (layer "F.Cu") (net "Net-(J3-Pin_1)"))
 (segment (start 98.5 147) (end 98.5 137) (width 1) (layer "F.Cu") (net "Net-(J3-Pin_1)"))
 (segment (start 102.5 136.4375) (end 108 136.4375) (width 1) (layer "F.Cu") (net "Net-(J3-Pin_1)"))
 (segment (start 110.9375 136.4375) (end 114.2 139.7) (width 1) (layer "F.Cu") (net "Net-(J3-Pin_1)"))
 (segment (start 83.04 50.96) (end 93.46 50.96) (width 1) (layer "F.Cu") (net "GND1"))
 (segment (start 99.5 55.08) (end 106.8 62.38) (width 1) (layer "F.Cu") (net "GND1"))
 (segment (start 119 142.65) (end 118.8 142.85) (width 1) (layer "F.Cu") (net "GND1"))
 (segment (start 102.5 139.5625) (end 108 139.5625) (width 1) (layer "F.Cu") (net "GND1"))
 (segment (start 175.04 92.04) (end 175.04 98.96) (width 1) (layer "F.Cu") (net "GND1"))
 (segment (start 106.8 62.38) (end 106.8 65.65) (width 1) (layer "F.Cu") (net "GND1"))
 (segment (start 121.85 142.85) (end 125 146) (width 1) (layer "F.Cu") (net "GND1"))
 (segment (start 119 140) (end 119 142.65) (width 1) (layer "F.Cu") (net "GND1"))
 (segment (start 132.2 65.65) (end 142.65 65.65) (width 1) (layer "F.Cu") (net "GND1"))
 (segment (start 108 139.5625) (end 108 141) (width 1) (layer "F.Cu") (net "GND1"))
 (segment (start 135.4375 139.5625) (end 135.5 139.5) (width 1) (layer "F.Cu") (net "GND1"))
 (segment (start 157 80) (end 163 80) (width 1) (layer "F.Cu") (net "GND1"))
 (segment (start 93.46 50.96) (end 94.42 50) (width 1) (layer "F.Cu") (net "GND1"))
 (segment (start 163 80) (end 175.04 92.04) (width 1) (layer "F.Cu") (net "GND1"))
 (segment (start 118.8 142.85) (end 121.85 142.85) (width 1) (layer "F.Cu") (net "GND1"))
 (segment (start 129 142) (end 125 146) (width 1) (layer "F.Cu") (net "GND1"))
 (segment (start 108 141) (end 109.5 142.5) (width 1) (layer "F.Cu") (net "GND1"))
 (segment (start 129 139.5625) (end 135.4375 139.5625) (width 1) (layer "F.Cu") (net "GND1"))
 (segment (start 129 139.5625) (end 129 142) (width 1) (layer "F.Cu") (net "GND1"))
 (segment (start 142.65 65.65) (end 157 80) (width 1) (layer "F.Cu") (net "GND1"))
 (via (at 125 146) (size 0.6) (drill 0.3) (layers "F.Cu" "B.Cu") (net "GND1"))
 (via (at 119 140) (size 0.6) (drill 0.3) (layers "F.Cu" "B.Cu") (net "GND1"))
 (via (at 109.5 142.5) (size 0.6) (drill 0.3) (layers "F.Cu" "B.Cu") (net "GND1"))
 (segment (start 125 161) (end 121.1725 161) (width 1) (layer "B.Cu") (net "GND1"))
 (segment (start 109.5 142.5) (end 112 140) (width 1) (layer "B.Cu") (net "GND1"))
 (segment (start 112 140) (end 119 140) (width 1) (layer "B.Cu") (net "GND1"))
 (segment (start 125 146) (end 125 161) (width 1) (layer "B.Cu") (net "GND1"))
 (segment (start 121.1725 161) (end 118.5 163.6725) (width 1) (layer "B.Cu") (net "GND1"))
 (segment (start 135.5 136.5) (end 149.5 136.5) (width 1) (layer "F.Cu") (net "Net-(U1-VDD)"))
 (segment (start 149.5 136.5) (end 159.5 126.5) (width 1) (layer "F.Cu") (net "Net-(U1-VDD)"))
 (segment (start 135.4375 136.4375) (end 135.5 136.375) (width 1) (layer "F.Cu") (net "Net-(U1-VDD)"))
 (segment (start 129 136.4375) (end 135.4375 136.4375) (width 1) (layer "F.Cu") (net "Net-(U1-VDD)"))
 (segment (start 172 126.5) (end 172 117) (width 1) (layer "F.Cu") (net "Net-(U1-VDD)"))
 (segment (start 116.5 138.5) (end 118.5625 136.4375) (width 1) (layer "F.Cu") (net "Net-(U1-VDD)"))
 (segment (start 172 117) (end 176 113) (width 1) (layer "F.Cu") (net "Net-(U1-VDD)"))
 (segment (start 116.5 142.85) (end 116.5 138.5) (width 1) (layer "F.Cu") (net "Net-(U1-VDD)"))
 (segment (start 176 102.46) (end 175.04 101.5) (width 1) (layer "F.Cu") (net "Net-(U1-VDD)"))
 (segment (start 118.5625 136.4375) (end 129 136.4375) (width 1) (layer "F.Cu") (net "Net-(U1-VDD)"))
 (segment (start 159.5 126.5) (end 172 126.5) (width 1) (layer "F.Cu") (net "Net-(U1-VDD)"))
 (segment (start 176 113) (end 176 102.46) (width 1) (layer "F.Cu") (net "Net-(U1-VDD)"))
 (segment (start 169 91) (end 172.5 94.5) (width 1) (layer "F.Cu") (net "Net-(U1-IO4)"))
 (segment (start 139.37 96.13) (end 142 93.5) (width 1) (layer "F.Cu") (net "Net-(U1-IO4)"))
 (segment (start 164 91) (end 169 91) (width 1) (layer "F.Cu") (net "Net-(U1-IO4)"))
 (segment (start 172.5 94.5) (end 172.5 98.96) (width 1) (layer "F.Cu") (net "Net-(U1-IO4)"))
 (segment (start 132.2 96.13) (end 139.37 96.13) (width 1) (layer "F.Cu") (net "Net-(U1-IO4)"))
 (via (at 142 93.5) (size 0.6) (drill 0.3) (layers "F.Cu" "B.Cu") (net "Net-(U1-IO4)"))
 (via (at 164 91) (size 0.6) (drill 0.3) (layers "F.Cu" "B.Cu") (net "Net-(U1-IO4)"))
 (segment (start 163 90) (end 164 91) (width 1) (layer "B.Cu") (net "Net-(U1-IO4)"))
 (segment (start 145.5 90) (end 163 90) (width 1) (layer "B.Cu") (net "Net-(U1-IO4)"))
 (segment (start 142 93.5) (end 145.5 90) (width 1) (layer "B.Cu") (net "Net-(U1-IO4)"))
 (segment (start 149.5 95) (end 143.01 88.51) (width 1) (layer "F.Cu") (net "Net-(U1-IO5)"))
 (segment (start 149.5 99.5) (end 149.5 95) (width 1) (layer "F.Cu") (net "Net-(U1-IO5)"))
 (segment (start 160 110) (end 149.5 99.5) (width 1) (layer "F.Cu") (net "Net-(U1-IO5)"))
 (segment (start 172.5 108) (end 170.5 110) (width 1) (layer "F.Cu") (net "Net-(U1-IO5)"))
 (segment (start 170.5 110) (end 160 110) (width 1) (layer "F.Cu") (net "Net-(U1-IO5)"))
 (segment (start 172.5 101.5) (end 172.5 108) (width 1) (layer "F.Cu") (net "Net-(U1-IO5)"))
 (segment (start 143.01 88.51) (end 132.2 88.51) (width 1) (layer "F.Cu") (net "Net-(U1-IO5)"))
 (segment (start 169 95) (end 161 95) (width 1) (layer "F.Cu") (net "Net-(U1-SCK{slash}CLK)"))
 (segment (start 140.13 111.37) (end 142 109.5) (width 1) (layer "F.Cu") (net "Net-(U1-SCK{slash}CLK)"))
 (segment (start 132.2 111.37) (end 140.13 111.37) (width 1) (layer "F.Cu") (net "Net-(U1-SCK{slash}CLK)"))
 (segment (start 142 109.5) (end 142 101.5) (width 1) (layer "F.Cu") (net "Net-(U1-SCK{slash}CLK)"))
 (segment (start 169.96 95.96) (end 169 95) (width 1) (layer "F.Cu") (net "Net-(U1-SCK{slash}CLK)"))
 (segment (start 161 95) (end 160 96) (width 1) (layer "F.Cu") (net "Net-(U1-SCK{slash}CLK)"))
 (segment (start 169.96 98.96) (end 169.96 95.96) (width 1) (layer "F.Cu") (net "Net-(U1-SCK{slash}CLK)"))
 (via (at 142 101.5) (size 0.6) (drill 0.3) (layers "F.Cu" "B.Cu") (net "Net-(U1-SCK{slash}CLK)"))
 (via (at 160 96) (size 0.6) (drill 0.3) (layers "F.Cu" "B.Cu") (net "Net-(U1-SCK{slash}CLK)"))
 (segment (start 146 96) (end 160 96) (width 1) (layer "B.Cu") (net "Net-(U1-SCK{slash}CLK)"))
 (segment (start 142 101.5) (end 142 100) (width 1) (layer "B.Cu") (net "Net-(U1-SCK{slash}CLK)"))
 (segment (start 142 100) (end 146 96) (width 1) (layer "B.Cu") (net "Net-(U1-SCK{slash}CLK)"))
 (segment (start 162.5 106) (end 162.5 103) (width 1) (layer "F.Cu") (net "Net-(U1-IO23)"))
 (segment (start 149.5 78) (end 144 78) (width 1) (layer "F.Cu") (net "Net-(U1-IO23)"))
 (segment (start 169.96 101.5) (end 169.96 105.54) (width 1) (layer "F.Cu") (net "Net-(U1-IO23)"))
 (segment (start 169.5 106) (end 162.5 106) (width 1) (layer "F.Cu") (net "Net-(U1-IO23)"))
 (segment (start 162.5 103) (end 149.5 90) (width 1) (layer "F.Cu") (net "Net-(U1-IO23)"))
 (segment (start 149.5 90) (end 149.5 78) (width 1) (layer "F.Cu") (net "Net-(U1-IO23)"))
 (segment (start 169.96 105.54) (end 169.5 106) (width 1) (layer "F.Cu") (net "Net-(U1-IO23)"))
 (segment (start 144 78) (end 134.19 68.19) (width 1) (layer "F.Cu") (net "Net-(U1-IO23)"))
 (segment (start 134.19 68.19) (end 132.2 68.19) (width 1) (layer "F.Cu") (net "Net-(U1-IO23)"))
 (segment (start 166.46 98) (end 163.5 98) (width 1) (layer "F.Cu") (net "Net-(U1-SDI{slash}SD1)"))
 (segment (start 135.29 106.29) (end 137 108) (width 1) (layer "F.Cu") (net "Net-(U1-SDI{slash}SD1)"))
 (segment (start 132.2 106.29) (end 135.29 106.29) (width 1) (layer "F.Cu") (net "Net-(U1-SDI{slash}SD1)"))
 (via (at 163.5 98) (size 0.6) (drill 0.3) (layers "F.Cu" "B.Cu") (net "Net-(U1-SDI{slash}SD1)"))
 (via (at 137 108) (size 0.6) (drill 0.3) (layers "F.Cu" "B.Cu") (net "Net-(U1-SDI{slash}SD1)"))
 (segment (start 157.5 103.5) (end 157.5 100.5) (width 1) (layer "B.Cu") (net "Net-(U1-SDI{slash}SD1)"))
 (segment (start 157.5 100.5) (end 160 98) (width 1) (layer "B.Cu") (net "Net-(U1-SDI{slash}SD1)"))
 (segment (start 160 98) (end 163.5 98) (width 1) (layer "B.Cu") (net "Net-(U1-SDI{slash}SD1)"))
 (segment (start 138 109) (end 152 109) (width 1) (layer "B.Cu") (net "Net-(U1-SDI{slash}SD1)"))
 (segment (start 152 109) (end 157.5 103.5) (width 1) (layer "B.Cu") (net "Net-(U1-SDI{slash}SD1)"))
 (segment (start 137 108) (end 138 109) (width 1) (layer "B.Cu") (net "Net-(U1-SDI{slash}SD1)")))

